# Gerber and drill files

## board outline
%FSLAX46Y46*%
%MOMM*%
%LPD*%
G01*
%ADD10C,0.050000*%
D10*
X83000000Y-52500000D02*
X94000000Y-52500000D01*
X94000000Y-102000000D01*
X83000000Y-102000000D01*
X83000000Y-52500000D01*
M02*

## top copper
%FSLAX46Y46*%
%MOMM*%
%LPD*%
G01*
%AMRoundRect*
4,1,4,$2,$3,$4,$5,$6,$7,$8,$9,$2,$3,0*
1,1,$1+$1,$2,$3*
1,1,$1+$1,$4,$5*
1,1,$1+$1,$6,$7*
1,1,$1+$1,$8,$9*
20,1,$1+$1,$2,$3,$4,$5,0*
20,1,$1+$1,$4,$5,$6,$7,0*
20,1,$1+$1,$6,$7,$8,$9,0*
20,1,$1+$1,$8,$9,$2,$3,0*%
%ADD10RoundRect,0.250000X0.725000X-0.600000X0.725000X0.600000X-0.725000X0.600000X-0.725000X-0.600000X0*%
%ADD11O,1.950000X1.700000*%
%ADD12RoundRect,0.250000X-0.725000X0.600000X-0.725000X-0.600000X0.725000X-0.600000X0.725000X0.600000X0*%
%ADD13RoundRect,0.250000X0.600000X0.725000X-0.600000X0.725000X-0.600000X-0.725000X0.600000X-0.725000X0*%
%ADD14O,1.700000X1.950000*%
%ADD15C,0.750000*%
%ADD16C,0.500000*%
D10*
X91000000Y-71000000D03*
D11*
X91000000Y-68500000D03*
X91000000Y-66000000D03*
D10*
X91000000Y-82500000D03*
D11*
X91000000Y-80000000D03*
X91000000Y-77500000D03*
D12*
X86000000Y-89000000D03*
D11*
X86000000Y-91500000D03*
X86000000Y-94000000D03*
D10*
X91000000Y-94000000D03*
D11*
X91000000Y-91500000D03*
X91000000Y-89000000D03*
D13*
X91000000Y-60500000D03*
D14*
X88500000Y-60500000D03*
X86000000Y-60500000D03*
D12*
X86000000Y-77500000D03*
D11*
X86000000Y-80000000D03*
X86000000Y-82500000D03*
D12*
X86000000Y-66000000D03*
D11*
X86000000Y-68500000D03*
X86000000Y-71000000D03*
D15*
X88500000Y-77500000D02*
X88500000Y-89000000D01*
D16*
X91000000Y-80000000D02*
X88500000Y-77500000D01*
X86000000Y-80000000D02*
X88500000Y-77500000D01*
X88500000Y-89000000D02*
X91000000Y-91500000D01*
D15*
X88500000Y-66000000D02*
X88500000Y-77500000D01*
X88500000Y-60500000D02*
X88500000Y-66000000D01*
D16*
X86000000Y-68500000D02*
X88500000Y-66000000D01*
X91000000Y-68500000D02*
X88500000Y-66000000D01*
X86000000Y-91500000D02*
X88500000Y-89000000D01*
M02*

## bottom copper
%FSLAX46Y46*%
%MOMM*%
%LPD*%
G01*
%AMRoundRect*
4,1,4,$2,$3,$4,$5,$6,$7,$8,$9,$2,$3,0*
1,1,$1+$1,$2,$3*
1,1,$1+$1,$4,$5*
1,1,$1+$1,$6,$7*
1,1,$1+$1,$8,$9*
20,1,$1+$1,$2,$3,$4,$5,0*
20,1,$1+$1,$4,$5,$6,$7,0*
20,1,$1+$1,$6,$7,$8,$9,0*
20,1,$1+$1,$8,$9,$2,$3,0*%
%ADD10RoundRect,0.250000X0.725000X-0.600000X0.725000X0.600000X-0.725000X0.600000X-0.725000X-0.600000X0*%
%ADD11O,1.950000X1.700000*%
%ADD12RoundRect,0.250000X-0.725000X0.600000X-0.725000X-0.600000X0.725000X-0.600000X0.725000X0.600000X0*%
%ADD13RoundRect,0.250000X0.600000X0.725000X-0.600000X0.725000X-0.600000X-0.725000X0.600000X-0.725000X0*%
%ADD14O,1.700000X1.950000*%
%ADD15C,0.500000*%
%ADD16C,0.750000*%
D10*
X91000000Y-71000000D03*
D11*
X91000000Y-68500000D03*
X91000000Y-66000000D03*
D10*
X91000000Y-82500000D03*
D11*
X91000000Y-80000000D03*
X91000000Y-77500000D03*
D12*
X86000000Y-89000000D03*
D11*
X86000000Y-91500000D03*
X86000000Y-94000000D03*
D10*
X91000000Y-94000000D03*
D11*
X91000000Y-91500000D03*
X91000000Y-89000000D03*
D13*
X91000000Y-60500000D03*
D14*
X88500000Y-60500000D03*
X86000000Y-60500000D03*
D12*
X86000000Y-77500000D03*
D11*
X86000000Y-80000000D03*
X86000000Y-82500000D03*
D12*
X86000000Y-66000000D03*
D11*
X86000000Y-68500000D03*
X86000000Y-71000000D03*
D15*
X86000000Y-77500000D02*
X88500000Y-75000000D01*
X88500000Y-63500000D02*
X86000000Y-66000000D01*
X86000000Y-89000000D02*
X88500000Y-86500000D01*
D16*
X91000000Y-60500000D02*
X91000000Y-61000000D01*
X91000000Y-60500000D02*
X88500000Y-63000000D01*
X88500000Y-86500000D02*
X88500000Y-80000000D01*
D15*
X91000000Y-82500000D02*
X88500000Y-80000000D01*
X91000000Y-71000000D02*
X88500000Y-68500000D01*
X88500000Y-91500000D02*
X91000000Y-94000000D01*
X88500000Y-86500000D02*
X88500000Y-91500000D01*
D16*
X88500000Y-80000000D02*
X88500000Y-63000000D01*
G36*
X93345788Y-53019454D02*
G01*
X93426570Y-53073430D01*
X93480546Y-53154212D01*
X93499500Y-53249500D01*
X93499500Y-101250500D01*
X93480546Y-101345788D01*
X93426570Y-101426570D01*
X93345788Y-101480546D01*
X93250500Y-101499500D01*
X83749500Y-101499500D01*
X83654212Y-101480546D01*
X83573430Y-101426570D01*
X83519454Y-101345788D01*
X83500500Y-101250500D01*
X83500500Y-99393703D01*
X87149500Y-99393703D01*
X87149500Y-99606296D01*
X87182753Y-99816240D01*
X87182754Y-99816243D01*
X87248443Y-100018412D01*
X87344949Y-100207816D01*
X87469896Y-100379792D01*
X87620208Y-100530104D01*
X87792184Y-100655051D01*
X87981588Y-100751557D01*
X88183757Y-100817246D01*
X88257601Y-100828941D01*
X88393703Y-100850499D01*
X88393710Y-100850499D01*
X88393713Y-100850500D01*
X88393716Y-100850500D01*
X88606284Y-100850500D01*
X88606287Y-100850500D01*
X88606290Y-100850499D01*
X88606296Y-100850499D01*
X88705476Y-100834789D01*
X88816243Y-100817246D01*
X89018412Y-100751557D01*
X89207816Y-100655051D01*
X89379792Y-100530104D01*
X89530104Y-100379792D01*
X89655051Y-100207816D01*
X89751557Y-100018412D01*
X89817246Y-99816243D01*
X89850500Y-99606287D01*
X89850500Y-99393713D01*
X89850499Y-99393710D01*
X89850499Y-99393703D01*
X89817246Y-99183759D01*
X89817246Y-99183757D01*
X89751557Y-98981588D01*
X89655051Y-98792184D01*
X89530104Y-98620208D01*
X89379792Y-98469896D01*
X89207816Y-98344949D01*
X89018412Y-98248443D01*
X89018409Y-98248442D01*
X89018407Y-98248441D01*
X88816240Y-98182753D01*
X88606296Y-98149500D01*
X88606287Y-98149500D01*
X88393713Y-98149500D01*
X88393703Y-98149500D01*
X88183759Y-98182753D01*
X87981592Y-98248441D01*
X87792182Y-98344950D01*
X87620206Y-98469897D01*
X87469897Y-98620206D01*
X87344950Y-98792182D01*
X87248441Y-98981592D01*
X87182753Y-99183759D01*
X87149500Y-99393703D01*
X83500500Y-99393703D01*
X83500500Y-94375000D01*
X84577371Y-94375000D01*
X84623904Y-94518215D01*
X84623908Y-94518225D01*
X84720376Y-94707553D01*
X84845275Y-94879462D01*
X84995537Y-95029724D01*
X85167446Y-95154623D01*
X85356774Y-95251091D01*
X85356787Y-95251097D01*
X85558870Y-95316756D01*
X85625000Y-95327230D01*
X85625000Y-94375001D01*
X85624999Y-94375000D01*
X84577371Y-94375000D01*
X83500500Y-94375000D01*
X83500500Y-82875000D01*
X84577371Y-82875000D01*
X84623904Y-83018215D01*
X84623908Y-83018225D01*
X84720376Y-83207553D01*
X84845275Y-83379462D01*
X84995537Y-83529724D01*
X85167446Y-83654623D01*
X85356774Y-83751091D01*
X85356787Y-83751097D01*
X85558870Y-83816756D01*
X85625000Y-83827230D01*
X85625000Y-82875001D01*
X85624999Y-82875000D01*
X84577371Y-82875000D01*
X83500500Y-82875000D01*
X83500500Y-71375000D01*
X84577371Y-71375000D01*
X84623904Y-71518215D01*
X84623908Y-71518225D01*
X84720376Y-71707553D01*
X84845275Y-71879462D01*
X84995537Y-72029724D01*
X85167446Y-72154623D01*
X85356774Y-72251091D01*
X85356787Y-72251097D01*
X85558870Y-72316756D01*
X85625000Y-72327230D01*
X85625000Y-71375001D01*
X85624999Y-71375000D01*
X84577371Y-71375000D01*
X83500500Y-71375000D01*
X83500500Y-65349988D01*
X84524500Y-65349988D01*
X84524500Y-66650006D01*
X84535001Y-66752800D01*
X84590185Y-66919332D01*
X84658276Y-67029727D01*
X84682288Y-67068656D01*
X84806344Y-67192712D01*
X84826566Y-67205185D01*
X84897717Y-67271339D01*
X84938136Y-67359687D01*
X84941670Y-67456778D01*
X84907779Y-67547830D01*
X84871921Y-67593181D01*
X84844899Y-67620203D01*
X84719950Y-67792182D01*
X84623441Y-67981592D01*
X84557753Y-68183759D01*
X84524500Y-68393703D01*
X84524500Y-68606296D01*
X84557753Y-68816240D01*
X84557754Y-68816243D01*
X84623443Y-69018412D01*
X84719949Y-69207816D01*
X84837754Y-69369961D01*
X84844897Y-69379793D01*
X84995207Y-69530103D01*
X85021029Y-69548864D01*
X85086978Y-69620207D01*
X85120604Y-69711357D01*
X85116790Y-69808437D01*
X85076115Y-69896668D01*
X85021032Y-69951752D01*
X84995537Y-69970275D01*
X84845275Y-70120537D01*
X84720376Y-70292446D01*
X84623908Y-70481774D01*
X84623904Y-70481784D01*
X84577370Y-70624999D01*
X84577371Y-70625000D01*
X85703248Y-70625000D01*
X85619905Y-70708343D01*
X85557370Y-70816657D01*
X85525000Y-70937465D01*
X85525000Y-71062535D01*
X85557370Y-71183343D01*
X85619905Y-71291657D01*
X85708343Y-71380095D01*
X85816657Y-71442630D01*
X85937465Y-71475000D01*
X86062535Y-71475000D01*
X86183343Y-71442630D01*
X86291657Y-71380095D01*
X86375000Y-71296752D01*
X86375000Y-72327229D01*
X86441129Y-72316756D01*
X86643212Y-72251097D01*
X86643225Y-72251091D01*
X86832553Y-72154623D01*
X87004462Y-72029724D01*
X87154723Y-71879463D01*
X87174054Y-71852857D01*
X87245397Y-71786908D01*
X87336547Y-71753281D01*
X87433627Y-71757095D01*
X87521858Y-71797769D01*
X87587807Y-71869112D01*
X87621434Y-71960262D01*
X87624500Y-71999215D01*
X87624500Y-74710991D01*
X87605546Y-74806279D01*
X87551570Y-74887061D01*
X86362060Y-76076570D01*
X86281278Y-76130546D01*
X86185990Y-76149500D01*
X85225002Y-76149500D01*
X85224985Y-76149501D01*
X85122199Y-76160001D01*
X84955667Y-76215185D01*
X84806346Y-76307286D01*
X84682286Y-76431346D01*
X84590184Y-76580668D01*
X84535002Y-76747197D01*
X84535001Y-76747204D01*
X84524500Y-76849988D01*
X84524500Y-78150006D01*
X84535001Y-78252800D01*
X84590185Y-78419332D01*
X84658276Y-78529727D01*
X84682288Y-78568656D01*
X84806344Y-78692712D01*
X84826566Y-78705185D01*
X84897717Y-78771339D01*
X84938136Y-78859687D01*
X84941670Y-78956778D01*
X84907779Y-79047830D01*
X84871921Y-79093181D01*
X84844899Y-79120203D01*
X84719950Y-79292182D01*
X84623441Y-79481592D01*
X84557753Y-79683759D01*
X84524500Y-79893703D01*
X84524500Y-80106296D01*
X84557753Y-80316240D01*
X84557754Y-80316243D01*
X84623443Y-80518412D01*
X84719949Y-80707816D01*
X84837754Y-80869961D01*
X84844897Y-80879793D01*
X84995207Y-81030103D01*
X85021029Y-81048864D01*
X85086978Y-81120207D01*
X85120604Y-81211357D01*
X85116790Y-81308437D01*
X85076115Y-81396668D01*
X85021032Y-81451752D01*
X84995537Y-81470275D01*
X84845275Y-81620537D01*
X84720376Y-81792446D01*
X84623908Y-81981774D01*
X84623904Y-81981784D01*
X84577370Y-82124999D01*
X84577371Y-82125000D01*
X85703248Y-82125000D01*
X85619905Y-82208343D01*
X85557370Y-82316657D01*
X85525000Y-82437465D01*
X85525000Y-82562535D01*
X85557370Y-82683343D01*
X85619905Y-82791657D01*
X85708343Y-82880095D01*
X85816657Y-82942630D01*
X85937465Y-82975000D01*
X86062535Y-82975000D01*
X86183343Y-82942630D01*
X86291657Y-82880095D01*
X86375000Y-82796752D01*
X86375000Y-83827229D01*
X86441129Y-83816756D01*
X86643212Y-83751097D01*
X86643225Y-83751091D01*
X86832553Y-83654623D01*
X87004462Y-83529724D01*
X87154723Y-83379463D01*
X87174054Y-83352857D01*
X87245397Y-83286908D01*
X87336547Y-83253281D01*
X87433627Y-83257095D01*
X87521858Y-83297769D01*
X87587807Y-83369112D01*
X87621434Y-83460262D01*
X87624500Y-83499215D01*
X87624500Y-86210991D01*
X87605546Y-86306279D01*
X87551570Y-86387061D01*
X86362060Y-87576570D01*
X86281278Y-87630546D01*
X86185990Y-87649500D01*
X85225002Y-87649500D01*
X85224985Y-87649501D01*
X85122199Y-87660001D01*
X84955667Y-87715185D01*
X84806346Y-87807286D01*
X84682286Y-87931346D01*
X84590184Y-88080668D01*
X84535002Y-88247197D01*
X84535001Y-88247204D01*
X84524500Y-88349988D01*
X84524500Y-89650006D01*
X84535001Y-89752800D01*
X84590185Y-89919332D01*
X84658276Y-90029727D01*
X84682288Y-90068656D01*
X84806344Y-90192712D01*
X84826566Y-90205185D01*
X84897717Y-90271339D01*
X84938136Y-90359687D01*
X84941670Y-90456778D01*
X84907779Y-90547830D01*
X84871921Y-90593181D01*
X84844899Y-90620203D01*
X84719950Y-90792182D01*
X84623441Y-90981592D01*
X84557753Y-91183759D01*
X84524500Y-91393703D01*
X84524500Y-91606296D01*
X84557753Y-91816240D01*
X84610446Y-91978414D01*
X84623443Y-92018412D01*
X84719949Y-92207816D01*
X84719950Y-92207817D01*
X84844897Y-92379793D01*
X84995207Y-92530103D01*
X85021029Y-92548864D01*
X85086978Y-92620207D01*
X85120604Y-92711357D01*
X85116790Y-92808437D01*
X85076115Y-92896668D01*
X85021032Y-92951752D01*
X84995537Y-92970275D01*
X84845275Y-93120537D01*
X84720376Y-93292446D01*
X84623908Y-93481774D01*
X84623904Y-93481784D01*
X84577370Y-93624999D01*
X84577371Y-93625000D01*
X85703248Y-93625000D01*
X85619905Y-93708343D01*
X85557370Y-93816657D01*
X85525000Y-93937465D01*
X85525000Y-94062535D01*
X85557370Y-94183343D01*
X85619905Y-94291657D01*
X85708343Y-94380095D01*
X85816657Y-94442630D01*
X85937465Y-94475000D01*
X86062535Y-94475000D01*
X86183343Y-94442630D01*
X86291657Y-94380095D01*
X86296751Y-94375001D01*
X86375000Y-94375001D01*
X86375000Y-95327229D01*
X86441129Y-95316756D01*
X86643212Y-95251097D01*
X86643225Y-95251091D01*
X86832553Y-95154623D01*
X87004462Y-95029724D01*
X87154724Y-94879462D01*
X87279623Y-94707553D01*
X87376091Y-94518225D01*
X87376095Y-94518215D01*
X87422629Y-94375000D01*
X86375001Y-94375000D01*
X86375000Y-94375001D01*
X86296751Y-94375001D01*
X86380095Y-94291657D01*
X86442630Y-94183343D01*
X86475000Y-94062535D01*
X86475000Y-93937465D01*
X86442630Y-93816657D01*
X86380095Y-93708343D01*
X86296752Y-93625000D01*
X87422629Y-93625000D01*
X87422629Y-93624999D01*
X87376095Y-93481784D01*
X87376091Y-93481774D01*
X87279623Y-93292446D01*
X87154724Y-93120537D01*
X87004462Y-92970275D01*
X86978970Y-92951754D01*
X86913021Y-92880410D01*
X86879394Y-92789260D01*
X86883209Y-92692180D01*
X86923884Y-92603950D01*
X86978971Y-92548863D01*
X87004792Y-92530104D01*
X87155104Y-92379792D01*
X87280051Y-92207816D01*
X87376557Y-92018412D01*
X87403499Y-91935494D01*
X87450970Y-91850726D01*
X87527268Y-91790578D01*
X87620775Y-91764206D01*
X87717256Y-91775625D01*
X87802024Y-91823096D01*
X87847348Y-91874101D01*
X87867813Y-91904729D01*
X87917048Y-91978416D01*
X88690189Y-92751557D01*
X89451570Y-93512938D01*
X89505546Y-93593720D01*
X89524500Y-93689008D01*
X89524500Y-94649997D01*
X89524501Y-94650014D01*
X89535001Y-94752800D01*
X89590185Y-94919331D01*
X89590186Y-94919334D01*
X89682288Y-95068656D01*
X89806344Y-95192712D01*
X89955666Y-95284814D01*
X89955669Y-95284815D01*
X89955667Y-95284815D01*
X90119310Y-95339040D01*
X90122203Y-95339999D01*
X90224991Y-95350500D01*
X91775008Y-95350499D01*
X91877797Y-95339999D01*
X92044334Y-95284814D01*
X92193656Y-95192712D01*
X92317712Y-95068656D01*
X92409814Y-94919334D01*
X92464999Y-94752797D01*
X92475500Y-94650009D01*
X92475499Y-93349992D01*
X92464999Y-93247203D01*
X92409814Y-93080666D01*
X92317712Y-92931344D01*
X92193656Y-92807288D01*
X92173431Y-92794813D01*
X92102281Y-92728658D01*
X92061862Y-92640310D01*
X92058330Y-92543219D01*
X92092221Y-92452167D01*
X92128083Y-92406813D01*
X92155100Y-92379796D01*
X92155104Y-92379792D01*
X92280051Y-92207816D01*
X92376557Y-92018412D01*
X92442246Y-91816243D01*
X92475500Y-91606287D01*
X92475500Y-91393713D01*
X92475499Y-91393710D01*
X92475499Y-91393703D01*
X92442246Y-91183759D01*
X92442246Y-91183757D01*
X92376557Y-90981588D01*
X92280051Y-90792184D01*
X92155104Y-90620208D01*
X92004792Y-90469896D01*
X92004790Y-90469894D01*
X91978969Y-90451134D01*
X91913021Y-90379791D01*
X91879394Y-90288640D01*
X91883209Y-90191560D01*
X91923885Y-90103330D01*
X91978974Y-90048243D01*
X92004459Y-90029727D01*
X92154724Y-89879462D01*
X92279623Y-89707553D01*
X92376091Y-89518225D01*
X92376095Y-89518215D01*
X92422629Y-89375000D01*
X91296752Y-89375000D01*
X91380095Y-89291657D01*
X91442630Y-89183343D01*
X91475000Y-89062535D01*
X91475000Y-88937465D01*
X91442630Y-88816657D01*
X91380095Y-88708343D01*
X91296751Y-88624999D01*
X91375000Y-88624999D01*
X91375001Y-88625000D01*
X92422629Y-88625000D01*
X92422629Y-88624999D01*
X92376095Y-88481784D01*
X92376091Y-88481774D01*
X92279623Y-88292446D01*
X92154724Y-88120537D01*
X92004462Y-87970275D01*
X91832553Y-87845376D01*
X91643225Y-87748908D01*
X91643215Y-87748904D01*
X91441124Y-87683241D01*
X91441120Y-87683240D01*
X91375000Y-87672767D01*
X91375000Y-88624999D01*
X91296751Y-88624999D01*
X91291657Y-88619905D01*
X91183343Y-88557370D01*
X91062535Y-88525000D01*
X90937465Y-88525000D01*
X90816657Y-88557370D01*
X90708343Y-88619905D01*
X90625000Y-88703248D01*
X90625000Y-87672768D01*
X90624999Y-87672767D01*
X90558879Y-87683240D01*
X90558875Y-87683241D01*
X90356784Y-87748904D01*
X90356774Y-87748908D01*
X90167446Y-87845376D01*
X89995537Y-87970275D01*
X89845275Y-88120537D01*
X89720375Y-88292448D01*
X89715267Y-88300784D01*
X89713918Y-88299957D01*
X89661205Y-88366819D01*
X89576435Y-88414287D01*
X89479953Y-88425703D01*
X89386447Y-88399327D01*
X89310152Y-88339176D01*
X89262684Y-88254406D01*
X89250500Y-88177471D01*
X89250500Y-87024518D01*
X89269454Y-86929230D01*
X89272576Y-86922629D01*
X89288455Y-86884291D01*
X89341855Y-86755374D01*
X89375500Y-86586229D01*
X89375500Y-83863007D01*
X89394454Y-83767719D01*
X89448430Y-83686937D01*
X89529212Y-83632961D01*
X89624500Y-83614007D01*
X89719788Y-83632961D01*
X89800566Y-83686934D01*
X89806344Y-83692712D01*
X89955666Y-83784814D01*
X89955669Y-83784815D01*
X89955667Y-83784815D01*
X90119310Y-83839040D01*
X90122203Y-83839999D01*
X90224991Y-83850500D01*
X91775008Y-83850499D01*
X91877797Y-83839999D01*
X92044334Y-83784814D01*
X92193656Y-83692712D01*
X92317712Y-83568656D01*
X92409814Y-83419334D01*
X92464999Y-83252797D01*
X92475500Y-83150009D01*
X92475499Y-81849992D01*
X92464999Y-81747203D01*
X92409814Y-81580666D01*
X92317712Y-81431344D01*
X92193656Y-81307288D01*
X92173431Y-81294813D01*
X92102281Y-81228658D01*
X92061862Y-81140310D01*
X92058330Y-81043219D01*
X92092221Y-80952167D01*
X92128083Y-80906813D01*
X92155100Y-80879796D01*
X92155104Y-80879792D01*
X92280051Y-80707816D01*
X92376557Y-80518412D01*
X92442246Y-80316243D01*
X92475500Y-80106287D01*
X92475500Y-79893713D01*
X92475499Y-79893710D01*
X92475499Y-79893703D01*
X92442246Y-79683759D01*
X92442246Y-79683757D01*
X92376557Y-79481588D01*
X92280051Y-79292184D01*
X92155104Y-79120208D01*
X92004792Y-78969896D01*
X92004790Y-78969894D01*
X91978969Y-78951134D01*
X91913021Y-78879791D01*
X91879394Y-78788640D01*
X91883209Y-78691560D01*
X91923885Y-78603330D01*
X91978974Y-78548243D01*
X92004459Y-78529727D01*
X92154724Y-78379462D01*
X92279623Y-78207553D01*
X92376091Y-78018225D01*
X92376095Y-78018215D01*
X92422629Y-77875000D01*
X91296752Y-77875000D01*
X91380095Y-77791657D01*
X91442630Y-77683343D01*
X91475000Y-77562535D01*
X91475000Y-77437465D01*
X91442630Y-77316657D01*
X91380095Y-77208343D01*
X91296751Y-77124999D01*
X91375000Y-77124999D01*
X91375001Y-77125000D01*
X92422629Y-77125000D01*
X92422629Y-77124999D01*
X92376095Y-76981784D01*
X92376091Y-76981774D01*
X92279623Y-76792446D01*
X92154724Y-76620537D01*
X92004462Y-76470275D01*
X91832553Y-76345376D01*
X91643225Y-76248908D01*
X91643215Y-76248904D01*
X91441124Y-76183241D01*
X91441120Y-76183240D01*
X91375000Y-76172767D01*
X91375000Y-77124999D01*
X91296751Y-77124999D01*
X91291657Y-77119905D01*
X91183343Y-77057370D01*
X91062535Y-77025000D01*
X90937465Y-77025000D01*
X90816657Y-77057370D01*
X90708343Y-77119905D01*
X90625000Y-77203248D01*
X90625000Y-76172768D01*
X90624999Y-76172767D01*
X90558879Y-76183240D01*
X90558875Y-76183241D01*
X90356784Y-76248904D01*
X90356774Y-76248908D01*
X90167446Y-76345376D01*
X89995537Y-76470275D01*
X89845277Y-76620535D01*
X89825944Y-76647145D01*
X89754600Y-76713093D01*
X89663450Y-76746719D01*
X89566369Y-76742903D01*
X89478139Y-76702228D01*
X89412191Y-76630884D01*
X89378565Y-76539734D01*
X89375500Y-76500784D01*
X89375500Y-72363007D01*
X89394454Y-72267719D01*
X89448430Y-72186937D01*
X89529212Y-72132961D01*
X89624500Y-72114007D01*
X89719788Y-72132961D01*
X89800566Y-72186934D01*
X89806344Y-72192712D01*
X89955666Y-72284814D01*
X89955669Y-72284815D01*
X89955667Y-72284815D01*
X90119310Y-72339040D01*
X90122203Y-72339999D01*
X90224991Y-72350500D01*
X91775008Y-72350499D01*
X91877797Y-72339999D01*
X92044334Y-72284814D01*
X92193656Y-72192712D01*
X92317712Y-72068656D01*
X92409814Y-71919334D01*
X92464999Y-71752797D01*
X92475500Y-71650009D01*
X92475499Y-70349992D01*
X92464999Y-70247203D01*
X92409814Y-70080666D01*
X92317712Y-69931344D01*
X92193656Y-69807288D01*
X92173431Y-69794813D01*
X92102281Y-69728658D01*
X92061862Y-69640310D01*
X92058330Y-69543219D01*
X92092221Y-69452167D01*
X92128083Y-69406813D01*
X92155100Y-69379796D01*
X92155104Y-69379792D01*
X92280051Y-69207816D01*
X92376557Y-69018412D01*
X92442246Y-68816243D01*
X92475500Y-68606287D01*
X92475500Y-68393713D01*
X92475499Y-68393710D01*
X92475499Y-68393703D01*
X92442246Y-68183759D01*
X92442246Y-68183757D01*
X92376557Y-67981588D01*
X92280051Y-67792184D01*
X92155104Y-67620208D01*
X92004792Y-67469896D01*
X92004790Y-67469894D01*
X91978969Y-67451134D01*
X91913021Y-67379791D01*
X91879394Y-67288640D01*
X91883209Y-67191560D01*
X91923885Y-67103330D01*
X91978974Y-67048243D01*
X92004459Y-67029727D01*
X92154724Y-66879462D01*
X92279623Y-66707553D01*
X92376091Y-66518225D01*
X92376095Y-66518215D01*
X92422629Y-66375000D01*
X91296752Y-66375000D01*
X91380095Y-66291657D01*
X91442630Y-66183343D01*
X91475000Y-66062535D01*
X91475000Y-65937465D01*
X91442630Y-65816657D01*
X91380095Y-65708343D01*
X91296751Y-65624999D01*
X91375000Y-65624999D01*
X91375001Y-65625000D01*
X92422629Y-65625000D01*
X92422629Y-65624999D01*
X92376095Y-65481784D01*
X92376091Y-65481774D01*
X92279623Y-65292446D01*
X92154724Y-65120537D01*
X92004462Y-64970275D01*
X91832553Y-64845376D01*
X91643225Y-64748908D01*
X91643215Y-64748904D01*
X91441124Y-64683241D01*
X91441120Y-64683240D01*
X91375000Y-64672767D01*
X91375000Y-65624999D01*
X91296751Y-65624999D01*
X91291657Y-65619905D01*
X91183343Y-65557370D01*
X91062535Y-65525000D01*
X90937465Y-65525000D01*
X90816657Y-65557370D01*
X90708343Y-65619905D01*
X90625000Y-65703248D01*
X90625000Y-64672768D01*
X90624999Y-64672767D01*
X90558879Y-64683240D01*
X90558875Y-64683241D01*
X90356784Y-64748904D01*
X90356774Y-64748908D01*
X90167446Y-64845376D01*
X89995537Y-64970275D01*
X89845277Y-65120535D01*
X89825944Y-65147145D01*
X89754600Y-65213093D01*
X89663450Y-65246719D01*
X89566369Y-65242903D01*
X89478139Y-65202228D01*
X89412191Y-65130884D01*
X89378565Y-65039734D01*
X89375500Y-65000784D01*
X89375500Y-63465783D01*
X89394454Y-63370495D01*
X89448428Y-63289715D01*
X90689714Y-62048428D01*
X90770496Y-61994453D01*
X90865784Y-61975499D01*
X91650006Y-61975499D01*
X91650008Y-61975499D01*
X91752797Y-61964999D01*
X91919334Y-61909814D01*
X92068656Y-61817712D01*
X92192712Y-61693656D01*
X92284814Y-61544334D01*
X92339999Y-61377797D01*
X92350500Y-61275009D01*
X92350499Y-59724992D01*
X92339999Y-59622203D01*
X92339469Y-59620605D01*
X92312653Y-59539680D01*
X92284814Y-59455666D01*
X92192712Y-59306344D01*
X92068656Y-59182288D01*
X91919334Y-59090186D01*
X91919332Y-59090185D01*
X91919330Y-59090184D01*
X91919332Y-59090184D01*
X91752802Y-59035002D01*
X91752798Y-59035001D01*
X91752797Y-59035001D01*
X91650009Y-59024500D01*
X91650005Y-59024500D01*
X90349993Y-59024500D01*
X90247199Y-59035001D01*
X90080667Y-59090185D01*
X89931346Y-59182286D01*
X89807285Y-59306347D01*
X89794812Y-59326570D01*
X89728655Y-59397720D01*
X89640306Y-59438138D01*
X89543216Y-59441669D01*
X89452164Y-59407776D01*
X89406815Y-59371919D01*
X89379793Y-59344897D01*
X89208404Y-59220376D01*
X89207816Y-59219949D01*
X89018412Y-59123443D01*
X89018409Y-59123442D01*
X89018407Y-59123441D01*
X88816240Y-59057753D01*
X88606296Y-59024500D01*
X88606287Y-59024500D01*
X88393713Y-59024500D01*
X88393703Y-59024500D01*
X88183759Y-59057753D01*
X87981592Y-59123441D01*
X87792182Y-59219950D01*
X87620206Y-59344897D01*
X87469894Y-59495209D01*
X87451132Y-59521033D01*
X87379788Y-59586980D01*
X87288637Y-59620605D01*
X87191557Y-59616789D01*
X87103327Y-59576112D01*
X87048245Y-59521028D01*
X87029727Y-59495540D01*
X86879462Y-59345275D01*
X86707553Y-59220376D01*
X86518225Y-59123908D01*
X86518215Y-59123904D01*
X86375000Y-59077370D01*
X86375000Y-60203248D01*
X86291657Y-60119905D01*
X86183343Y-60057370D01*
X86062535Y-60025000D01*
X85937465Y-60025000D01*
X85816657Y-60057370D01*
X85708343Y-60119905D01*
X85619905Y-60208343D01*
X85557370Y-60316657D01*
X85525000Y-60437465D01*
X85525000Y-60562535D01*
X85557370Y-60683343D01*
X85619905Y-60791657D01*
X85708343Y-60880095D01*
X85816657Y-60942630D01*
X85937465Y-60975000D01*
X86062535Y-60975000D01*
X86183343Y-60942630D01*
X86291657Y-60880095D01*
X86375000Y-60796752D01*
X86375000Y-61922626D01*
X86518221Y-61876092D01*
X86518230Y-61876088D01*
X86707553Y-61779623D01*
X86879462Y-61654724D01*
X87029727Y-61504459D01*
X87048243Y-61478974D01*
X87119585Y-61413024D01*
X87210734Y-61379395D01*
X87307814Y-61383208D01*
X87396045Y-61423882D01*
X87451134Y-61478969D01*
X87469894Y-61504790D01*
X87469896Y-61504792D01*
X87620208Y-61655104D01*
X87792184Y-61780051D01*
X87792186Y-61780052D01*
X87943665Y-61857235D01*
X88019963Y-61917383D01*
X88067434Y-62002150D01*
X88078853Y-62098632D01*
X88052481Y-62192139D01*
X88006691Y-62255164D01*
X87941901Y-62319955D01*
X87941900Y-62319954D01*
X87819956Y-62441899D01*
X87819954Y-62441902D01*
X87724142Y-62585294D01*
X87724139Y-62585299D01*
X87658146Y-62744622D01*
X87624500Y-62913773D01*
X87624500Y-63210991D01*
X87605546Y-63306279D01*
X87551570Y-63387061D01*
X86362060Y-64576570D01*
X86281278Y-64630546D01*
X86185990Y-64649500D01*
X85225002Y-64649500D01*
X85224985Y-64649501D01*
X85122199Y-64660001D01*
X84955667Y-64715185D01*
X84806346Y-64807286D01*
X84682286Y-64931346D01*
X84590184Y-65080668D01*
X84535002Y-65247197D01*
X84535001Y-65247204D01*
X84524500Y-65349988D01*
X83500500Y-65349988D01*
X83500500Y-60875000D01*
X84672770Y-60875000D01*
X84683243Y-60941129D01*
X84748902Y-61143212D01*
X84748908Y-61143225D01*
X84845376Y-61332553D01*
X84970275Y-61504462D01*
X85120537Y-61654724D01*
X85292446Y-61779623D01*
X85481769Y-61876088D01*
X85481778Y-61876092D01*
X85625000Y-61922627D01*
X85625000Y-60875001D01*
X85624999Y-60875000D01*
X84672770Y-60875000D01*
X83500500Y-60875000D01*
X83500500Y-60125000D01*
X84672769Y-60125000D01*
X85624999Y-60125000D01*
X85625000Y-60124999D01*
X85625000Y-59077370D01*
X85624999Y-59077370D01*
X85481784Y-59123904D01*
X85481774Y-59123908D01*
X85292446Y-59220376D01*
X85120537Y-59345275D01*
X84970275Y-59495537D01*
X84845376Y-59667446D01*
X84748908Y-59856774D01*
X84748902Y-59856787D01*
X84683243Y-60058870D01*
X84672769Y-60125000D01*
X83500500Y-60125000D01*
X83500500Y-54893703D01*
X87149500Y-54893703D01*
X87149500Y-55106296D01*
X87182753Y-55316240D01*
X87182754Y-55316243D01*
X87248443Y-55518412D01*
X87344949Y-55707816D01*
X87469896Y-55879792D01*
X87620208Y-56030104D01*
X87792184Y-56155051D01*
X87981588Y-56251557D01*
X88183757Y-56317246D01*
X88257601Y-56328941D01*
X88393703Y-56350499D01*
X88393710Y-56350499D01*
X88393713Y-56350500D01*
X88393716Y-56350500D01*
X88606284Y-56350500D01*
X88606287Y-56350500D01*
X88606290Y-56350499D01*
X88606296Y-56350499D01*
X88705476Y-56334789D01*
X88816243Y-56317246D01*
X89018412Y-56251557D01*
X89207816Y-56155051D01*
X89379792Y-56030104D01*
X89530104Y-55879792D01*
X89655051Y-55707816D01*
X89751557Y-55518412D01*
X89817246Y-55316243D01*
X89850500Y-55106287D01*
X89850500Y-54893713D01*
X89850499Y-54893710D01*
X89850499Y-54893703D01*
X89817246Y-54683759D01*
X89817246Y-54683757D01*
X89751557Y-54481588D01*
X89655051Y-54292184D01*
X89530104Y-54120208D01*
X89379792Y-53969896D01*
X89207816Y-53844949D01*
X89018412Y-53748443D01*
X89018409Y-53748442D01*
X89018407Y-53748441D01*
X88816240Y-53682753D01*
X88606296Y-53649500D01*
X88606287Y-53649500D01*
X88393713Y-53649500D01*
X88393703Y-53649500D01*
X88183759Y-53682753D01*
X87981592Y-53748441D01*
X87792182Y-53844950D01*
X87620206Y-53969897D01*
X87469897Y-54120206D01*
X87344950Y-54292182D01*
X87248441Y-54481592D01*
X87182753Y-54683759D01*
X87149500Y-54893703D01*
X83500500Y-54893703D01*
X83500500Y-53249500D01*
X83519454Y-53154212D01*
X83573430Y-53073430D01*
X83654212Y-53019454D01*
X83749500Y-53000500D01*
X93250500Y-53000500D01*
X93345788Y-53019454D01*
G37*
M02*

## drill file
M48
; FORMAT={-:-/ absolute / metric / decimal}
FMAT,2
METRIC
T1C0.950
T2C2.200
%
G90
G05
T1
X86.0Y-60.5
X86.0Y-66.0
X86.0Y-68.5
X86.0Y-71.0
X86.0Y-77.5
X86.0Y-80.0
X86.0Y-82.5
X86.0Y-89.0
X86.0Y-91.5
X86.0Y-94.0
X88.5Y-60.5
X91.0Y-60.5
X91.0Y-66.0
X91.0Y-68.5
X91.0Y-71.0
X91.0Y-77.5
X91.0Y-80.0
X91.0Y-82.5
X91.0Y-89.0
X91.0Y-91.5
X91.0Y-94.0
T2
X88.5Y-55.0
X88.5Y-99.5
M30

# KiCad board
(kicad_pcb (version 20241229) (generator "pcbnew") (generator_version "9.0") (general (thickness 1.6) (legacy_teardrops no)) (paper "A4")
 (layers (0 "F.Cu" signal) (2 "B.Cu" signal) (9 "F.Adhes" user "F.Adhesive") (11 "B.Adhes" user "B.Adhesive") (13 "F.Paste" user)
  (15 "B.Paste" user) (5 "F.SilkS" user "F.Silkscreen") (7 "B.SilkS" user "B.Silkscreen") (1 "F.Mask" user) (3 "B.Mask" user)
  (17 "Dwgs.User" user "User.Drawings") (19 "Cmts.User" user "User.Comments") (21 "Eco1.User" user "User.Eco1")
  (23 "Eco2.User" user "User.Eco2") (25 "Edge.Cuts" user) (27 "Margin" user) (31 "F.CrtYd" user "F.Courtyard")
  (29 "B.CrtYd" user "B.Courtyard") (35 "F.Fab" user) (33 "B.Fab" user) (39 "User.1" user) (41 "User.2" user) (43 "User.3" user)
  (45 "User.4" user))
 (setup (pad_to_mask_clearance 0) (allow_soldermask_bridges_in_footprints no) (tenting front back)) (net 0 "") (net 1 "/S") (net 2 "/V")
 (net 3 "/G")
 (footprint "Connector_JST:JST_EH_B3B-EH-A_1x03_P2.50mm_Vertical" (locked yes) (layer "F.Cu") (at 91 71 90)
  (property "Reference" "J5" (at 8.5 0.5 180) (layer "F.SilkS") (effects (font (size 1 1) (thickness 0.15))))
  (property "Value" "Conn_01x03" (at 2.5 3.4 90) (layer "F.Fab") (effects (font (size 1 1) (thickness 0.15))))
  (pad "1" thru_hole roundrect (at 0 0 90) (size 1.7 1.95) (drill 0.95) (layers "*.Cu" "*.Mask") (remove_unused_layers no)
   (roundrect_rratio 0.147059) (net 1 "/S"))
  (pad "2" thru_hole oval (at 2.5 0 90) (size 1.7 1.95) (drill 0.95) (layers "*.Cu" "*.Mask") (remove_unused_layers no) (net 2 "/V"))
  (pad "3" thru_hole oval (at 5 0 90) (size 1.7 1.95) (drill 0.95) (layers "*.Cu" "*.Mask") (remove_unused_layers no) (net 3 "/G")))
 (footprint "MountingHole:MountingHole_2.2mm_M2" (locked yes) (layer "F.Cu") (at 88.5 99.5)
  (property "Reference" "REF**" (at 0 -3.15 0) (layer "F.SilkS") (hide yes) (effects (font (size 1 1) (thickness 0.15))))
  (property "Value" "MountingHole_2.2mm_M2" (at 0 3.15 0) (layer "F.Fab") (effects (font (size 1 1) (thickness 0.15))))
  (pad "" np_thru_hole circle (at 0 0) (size 2.2 2.2) (drill 2.2) (layers "*.Cu" "*.Mask")))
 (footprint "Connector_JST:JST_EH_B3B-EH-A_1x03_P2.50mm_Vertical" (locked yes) (layer "F.Cu") (at 91 82.5 90)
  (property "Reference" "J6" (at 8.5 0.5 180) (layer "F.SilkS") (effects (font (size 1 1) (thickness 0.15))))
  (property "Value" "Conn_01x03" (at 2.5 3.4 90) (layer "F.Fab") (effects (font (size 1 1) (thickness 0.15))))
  (pad "1" thru_hole roundrect (at 0 0 90) (size 1.7 1.95) (drill 0.95) (layers "*.Cu" "*.Mask") (remove_unused_layers no)
   (roundrect_rratio 0.147059) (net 1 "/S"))
  (pad "2" thru_hole oval (at 2.5 0 90) (size 1.7 1.95) (drill 0.95) (layers "*.Cu" "*.Mask") (remove_unused_layers no) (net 2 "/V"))
  (pad "3" thru_hole oval (at 5 0 90) (size 1.7 1.95) (drill 0.95) (layers "*.Cu" "*.Mask") (remove_unused_layers no) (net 3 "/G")))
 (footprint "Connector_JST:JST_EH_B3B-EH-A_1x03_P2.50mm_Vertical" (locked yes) (layer "F.Cu") (at 86 89 -90)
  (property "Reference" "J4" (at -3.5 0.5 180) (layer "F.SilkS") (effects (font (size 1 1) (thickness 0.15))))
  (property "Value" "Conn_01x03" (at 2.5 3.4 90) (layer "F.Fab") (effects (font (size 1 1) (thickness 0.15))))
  (pad "1" thru_hole roundrect (at 0 0 270) (size 1.7 1.95) (drill 0.95) (layers "*.Cu" "*.Mask") (remove_unused_layers no)
   (roundrect_rratio 0.147059) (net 1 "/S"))
  (pad "2" thru_hole oval (at 2.5 0 270) (size 1.7 1.95) (drill 0.95) (layers "*.Cu" "*.Mask") (remove_unused_layers no) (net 2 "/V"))
  (pad "3" thru_hole oval (at 5 0 270) (size 1.7 1.95) (drill 0.95) (layers "*.Cu" "*.Mask") (remove_unused_layers no) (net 3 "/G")))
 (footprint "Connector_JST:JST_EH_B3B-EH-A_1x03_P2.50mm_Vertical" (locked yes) (layer "F.Cu") (at 91 94 90)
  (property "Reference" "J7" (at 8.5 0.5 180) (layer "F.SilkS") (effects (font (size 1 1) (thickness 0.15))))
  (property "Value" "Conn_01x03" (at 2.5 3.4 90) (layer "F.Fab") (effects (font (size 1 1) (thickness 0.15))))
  (pad "1" thru_hole roundrect (at 0 0 90) (size 1.7 1.95) (drill 0.95) (layers "*.Cu" "*.Mask") (remove_unused_layers no)
   (roundrect_rratio 0.147059) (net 1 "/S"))
  (pad "2" thru_hole oval (at 2.5 0 90) (size 1.7 1.95) (drill 0.95) (layers "*.Cu" "*.Mask") (remove_unused_layers no) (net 2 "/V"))
  (pad "3" thru_hole oval (at 5 0 90) (size 1.7 1.95) (drill 0.95) (layers "*.Cu" "*.Mask") (remove_unused_layers no) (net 3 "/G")))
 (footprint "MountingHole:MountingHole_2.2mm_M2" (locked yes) (layer "F.Cu") (at 88.5 55)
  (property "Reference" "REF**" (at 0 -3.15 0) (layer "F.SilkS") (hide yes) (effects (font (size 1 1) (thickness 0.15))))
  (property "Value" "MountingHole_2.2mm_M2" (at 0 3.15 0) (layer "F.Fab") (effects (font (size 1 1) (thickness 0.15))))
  (pad "" np_thru_hole circle (at 0 0) (size 2.2 2.2) (drill 2.2) (layers "*.Cu" "*.Mask")))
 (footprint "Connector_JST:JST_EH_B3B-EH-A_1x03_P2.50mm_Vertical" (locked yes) (layer "F.Cu") (at 91 60.5 180)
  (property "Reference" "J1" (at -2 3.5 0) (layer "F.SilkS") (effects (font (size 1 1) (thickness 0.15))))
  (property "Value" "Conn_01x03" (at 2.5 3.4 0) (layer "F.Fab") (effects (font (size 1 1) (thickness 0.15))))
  (pad "1" thru_hole roundrect (at 0 0 180) (size 1.7 1.95) (drill 0.95) (layers "*.Cu" "*.Mask") (remove_unused_layers no)
   (roundrect_rratio 0.147059) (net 1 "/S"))
  (pad "2" thru_hole oval (at 2.5 0 180) (size 1.7 1.95) (drill 0.95) (layers "*.Cu" "*.Mask") (remove_unused_layers no) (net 2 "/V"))
  (pad "3" thru_hole oval (at 5 0 180) (size 1.7 1.95) (drill 0.95) (layers "*.Cu" "*.Mask") (remove_unused_layers no) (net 3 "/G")))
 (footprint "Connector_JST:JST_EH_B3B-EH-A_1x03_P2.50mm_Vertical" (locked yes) (layer "F.Cu") (at 86 77.5 -90)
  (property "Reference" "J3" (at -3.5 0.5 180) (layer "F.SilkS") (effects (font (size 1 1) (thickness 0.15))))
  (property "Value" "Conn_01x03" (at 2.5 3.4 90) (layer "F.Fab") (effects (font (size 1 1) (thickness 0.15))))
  (pad "1" thru_hole roundrect (at 0 0 270) (size 1.7 1.95) (drill 0.95) (layers "*.Cu" "*.Mask") (remove_unused_layers no)
   (roundrect_rratio 0.147059) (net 1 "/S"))
  (pad "2" thru_hole oval (at 2.5 0 270) (size 1.7 1.95) (drill 0.95) (layers "*.Cu" "*.Mask") (remove_unused_layers no) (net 2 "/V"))
  (pad "3" thru_hole oval (at 5 0 270) (size 1.7 1.95) (drill 0.95) (layers "*.Cu" "*.Mask") (remove_unused_layers no) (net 3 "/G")))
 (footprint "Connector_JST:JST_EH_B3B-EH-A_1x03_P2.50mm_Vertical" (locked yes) (layer "F.Cu") (at 86 66 -90)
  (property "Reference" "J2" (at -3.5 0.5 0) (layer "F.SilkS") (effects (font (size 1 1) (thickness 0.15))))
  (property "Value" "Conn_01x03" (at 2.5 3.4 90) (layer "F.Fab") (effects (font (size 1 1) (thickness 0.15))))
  (pad "1" thru_hole roundrect (at 0 0 270) (size 1.7 1.95) (drill 0.95) (layers "*.Cu" "*.Mask") (remove_unused_layers no)
   (roundrect_rratio 0.147059) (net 1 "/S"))
  (pad "2" thru_hole oval (at 2.5 0 270) (size 1.7 1.95) (drill 0.95) (layers "*.Cu" "*.Mask") (remove_unused_layers no) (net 2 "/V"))
  (pad "3" thru_hole oval (at 5 0 270) (size 1.7 1.95) (drill 0.95) (layers "*.Cu" "*.Mask") (remove_unused_layers no) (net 3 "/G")))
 (gr_rect (start 83 52.5) (end 94 102) (stroke (width 0.05) (type default)) (fill no) (locked yes) (layer "Edge.Cuts"))
 (segment (start 86 77.5) (end 88.5 75) (width 0.5) (locked yes) (layer "B.Cu") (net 1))
 (segment (start 88.5 63.5) (end 86 66) (width 0.5) (locked yes) (layer "B.Cu") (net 1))
 (segment (start 86 89) (end 88.5 86.5) (width 0.5) (locked yes) (layer "B.Cu") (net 1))
 (segment (start 91 60.5) (end 91 61) (width 0.75) (locked yes) (layer "B.Cu") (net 1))
 (segment (start 91 60.5) (end 88.5 63) (width 0.75) (locked yes) (layer "B.Cu") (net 1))
 (segment (start 88.5 86.5) (end 88.5 80) (width 0.75) (locked yes) (layer "B.Cu") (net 1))
 (segment (start 91 82.5) (end 88.5 80) (width 0.5) (locked yes) (layer "B.Cu") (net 1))
 (segment (start 91 71) (end 88.5 68.5) (width 0.5) (locked yes) (layer "B.Cu") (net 1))
 (segment (start 88.5 91.5) (end 91 94) (width 0.5) (locked yes) (layer "B.Cu") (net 1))
 (segment (start 88.5 86.5) (end 88.5 91.5) (width 0.5) (locked yes) (layer "B.Cu") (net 1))
 (segment (start 88.5 80) (end 88.5 63) (width 0.75) (locked yes) (layer "B.Cu") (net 1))
 (segment (start 88.5 77.5) (end 88.5 89) (width 0.75) (locked yes) (layer "F.Cu") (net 2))
 (segment (start 91 80) (end 88.5 77.5) (width 0.5) (locked yes) (layer "F.Cu") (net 2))
 (segment (start 86 80) (end 88.5 77.5) (width 0.5) (locked yes) (layer "F.Cu") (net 2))
 (segment (start 88.5 89) (end 91 91.5) (width 0.5) (locked yes) (layer "F.Cu") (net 2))
 (segment (start 88.5 66) (end 88.5 77.5) (width 0.75) (locked yes) (layer "F.Cu") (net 2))
 (segment (start 88.5 60.5) (end 88.5 66) (width 0.75) (locked yes) (layer "F.Cu") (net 2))
 (segment (start 86 68.5) (end 88.5 66) (width 0.5) (locked yes) (layer "F.Cu") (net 2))
 (segment (start 91 68.5) (end 88.5 66) (width 0.5) (locked yes) (layer "F.Cu") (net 2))
 (segment (start 86 91.5) (end 88.5 89) (width 0.5) (locked yes) (layer "F.Cu") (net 2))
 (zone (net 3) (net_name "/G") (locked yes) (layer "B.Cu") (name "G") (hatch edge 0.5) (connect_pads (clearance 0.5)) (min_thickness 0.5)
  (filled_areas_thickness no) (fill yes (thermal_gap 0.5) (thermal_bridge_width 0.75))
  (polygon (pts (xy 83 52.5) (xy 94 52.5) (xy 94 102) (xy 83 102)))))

